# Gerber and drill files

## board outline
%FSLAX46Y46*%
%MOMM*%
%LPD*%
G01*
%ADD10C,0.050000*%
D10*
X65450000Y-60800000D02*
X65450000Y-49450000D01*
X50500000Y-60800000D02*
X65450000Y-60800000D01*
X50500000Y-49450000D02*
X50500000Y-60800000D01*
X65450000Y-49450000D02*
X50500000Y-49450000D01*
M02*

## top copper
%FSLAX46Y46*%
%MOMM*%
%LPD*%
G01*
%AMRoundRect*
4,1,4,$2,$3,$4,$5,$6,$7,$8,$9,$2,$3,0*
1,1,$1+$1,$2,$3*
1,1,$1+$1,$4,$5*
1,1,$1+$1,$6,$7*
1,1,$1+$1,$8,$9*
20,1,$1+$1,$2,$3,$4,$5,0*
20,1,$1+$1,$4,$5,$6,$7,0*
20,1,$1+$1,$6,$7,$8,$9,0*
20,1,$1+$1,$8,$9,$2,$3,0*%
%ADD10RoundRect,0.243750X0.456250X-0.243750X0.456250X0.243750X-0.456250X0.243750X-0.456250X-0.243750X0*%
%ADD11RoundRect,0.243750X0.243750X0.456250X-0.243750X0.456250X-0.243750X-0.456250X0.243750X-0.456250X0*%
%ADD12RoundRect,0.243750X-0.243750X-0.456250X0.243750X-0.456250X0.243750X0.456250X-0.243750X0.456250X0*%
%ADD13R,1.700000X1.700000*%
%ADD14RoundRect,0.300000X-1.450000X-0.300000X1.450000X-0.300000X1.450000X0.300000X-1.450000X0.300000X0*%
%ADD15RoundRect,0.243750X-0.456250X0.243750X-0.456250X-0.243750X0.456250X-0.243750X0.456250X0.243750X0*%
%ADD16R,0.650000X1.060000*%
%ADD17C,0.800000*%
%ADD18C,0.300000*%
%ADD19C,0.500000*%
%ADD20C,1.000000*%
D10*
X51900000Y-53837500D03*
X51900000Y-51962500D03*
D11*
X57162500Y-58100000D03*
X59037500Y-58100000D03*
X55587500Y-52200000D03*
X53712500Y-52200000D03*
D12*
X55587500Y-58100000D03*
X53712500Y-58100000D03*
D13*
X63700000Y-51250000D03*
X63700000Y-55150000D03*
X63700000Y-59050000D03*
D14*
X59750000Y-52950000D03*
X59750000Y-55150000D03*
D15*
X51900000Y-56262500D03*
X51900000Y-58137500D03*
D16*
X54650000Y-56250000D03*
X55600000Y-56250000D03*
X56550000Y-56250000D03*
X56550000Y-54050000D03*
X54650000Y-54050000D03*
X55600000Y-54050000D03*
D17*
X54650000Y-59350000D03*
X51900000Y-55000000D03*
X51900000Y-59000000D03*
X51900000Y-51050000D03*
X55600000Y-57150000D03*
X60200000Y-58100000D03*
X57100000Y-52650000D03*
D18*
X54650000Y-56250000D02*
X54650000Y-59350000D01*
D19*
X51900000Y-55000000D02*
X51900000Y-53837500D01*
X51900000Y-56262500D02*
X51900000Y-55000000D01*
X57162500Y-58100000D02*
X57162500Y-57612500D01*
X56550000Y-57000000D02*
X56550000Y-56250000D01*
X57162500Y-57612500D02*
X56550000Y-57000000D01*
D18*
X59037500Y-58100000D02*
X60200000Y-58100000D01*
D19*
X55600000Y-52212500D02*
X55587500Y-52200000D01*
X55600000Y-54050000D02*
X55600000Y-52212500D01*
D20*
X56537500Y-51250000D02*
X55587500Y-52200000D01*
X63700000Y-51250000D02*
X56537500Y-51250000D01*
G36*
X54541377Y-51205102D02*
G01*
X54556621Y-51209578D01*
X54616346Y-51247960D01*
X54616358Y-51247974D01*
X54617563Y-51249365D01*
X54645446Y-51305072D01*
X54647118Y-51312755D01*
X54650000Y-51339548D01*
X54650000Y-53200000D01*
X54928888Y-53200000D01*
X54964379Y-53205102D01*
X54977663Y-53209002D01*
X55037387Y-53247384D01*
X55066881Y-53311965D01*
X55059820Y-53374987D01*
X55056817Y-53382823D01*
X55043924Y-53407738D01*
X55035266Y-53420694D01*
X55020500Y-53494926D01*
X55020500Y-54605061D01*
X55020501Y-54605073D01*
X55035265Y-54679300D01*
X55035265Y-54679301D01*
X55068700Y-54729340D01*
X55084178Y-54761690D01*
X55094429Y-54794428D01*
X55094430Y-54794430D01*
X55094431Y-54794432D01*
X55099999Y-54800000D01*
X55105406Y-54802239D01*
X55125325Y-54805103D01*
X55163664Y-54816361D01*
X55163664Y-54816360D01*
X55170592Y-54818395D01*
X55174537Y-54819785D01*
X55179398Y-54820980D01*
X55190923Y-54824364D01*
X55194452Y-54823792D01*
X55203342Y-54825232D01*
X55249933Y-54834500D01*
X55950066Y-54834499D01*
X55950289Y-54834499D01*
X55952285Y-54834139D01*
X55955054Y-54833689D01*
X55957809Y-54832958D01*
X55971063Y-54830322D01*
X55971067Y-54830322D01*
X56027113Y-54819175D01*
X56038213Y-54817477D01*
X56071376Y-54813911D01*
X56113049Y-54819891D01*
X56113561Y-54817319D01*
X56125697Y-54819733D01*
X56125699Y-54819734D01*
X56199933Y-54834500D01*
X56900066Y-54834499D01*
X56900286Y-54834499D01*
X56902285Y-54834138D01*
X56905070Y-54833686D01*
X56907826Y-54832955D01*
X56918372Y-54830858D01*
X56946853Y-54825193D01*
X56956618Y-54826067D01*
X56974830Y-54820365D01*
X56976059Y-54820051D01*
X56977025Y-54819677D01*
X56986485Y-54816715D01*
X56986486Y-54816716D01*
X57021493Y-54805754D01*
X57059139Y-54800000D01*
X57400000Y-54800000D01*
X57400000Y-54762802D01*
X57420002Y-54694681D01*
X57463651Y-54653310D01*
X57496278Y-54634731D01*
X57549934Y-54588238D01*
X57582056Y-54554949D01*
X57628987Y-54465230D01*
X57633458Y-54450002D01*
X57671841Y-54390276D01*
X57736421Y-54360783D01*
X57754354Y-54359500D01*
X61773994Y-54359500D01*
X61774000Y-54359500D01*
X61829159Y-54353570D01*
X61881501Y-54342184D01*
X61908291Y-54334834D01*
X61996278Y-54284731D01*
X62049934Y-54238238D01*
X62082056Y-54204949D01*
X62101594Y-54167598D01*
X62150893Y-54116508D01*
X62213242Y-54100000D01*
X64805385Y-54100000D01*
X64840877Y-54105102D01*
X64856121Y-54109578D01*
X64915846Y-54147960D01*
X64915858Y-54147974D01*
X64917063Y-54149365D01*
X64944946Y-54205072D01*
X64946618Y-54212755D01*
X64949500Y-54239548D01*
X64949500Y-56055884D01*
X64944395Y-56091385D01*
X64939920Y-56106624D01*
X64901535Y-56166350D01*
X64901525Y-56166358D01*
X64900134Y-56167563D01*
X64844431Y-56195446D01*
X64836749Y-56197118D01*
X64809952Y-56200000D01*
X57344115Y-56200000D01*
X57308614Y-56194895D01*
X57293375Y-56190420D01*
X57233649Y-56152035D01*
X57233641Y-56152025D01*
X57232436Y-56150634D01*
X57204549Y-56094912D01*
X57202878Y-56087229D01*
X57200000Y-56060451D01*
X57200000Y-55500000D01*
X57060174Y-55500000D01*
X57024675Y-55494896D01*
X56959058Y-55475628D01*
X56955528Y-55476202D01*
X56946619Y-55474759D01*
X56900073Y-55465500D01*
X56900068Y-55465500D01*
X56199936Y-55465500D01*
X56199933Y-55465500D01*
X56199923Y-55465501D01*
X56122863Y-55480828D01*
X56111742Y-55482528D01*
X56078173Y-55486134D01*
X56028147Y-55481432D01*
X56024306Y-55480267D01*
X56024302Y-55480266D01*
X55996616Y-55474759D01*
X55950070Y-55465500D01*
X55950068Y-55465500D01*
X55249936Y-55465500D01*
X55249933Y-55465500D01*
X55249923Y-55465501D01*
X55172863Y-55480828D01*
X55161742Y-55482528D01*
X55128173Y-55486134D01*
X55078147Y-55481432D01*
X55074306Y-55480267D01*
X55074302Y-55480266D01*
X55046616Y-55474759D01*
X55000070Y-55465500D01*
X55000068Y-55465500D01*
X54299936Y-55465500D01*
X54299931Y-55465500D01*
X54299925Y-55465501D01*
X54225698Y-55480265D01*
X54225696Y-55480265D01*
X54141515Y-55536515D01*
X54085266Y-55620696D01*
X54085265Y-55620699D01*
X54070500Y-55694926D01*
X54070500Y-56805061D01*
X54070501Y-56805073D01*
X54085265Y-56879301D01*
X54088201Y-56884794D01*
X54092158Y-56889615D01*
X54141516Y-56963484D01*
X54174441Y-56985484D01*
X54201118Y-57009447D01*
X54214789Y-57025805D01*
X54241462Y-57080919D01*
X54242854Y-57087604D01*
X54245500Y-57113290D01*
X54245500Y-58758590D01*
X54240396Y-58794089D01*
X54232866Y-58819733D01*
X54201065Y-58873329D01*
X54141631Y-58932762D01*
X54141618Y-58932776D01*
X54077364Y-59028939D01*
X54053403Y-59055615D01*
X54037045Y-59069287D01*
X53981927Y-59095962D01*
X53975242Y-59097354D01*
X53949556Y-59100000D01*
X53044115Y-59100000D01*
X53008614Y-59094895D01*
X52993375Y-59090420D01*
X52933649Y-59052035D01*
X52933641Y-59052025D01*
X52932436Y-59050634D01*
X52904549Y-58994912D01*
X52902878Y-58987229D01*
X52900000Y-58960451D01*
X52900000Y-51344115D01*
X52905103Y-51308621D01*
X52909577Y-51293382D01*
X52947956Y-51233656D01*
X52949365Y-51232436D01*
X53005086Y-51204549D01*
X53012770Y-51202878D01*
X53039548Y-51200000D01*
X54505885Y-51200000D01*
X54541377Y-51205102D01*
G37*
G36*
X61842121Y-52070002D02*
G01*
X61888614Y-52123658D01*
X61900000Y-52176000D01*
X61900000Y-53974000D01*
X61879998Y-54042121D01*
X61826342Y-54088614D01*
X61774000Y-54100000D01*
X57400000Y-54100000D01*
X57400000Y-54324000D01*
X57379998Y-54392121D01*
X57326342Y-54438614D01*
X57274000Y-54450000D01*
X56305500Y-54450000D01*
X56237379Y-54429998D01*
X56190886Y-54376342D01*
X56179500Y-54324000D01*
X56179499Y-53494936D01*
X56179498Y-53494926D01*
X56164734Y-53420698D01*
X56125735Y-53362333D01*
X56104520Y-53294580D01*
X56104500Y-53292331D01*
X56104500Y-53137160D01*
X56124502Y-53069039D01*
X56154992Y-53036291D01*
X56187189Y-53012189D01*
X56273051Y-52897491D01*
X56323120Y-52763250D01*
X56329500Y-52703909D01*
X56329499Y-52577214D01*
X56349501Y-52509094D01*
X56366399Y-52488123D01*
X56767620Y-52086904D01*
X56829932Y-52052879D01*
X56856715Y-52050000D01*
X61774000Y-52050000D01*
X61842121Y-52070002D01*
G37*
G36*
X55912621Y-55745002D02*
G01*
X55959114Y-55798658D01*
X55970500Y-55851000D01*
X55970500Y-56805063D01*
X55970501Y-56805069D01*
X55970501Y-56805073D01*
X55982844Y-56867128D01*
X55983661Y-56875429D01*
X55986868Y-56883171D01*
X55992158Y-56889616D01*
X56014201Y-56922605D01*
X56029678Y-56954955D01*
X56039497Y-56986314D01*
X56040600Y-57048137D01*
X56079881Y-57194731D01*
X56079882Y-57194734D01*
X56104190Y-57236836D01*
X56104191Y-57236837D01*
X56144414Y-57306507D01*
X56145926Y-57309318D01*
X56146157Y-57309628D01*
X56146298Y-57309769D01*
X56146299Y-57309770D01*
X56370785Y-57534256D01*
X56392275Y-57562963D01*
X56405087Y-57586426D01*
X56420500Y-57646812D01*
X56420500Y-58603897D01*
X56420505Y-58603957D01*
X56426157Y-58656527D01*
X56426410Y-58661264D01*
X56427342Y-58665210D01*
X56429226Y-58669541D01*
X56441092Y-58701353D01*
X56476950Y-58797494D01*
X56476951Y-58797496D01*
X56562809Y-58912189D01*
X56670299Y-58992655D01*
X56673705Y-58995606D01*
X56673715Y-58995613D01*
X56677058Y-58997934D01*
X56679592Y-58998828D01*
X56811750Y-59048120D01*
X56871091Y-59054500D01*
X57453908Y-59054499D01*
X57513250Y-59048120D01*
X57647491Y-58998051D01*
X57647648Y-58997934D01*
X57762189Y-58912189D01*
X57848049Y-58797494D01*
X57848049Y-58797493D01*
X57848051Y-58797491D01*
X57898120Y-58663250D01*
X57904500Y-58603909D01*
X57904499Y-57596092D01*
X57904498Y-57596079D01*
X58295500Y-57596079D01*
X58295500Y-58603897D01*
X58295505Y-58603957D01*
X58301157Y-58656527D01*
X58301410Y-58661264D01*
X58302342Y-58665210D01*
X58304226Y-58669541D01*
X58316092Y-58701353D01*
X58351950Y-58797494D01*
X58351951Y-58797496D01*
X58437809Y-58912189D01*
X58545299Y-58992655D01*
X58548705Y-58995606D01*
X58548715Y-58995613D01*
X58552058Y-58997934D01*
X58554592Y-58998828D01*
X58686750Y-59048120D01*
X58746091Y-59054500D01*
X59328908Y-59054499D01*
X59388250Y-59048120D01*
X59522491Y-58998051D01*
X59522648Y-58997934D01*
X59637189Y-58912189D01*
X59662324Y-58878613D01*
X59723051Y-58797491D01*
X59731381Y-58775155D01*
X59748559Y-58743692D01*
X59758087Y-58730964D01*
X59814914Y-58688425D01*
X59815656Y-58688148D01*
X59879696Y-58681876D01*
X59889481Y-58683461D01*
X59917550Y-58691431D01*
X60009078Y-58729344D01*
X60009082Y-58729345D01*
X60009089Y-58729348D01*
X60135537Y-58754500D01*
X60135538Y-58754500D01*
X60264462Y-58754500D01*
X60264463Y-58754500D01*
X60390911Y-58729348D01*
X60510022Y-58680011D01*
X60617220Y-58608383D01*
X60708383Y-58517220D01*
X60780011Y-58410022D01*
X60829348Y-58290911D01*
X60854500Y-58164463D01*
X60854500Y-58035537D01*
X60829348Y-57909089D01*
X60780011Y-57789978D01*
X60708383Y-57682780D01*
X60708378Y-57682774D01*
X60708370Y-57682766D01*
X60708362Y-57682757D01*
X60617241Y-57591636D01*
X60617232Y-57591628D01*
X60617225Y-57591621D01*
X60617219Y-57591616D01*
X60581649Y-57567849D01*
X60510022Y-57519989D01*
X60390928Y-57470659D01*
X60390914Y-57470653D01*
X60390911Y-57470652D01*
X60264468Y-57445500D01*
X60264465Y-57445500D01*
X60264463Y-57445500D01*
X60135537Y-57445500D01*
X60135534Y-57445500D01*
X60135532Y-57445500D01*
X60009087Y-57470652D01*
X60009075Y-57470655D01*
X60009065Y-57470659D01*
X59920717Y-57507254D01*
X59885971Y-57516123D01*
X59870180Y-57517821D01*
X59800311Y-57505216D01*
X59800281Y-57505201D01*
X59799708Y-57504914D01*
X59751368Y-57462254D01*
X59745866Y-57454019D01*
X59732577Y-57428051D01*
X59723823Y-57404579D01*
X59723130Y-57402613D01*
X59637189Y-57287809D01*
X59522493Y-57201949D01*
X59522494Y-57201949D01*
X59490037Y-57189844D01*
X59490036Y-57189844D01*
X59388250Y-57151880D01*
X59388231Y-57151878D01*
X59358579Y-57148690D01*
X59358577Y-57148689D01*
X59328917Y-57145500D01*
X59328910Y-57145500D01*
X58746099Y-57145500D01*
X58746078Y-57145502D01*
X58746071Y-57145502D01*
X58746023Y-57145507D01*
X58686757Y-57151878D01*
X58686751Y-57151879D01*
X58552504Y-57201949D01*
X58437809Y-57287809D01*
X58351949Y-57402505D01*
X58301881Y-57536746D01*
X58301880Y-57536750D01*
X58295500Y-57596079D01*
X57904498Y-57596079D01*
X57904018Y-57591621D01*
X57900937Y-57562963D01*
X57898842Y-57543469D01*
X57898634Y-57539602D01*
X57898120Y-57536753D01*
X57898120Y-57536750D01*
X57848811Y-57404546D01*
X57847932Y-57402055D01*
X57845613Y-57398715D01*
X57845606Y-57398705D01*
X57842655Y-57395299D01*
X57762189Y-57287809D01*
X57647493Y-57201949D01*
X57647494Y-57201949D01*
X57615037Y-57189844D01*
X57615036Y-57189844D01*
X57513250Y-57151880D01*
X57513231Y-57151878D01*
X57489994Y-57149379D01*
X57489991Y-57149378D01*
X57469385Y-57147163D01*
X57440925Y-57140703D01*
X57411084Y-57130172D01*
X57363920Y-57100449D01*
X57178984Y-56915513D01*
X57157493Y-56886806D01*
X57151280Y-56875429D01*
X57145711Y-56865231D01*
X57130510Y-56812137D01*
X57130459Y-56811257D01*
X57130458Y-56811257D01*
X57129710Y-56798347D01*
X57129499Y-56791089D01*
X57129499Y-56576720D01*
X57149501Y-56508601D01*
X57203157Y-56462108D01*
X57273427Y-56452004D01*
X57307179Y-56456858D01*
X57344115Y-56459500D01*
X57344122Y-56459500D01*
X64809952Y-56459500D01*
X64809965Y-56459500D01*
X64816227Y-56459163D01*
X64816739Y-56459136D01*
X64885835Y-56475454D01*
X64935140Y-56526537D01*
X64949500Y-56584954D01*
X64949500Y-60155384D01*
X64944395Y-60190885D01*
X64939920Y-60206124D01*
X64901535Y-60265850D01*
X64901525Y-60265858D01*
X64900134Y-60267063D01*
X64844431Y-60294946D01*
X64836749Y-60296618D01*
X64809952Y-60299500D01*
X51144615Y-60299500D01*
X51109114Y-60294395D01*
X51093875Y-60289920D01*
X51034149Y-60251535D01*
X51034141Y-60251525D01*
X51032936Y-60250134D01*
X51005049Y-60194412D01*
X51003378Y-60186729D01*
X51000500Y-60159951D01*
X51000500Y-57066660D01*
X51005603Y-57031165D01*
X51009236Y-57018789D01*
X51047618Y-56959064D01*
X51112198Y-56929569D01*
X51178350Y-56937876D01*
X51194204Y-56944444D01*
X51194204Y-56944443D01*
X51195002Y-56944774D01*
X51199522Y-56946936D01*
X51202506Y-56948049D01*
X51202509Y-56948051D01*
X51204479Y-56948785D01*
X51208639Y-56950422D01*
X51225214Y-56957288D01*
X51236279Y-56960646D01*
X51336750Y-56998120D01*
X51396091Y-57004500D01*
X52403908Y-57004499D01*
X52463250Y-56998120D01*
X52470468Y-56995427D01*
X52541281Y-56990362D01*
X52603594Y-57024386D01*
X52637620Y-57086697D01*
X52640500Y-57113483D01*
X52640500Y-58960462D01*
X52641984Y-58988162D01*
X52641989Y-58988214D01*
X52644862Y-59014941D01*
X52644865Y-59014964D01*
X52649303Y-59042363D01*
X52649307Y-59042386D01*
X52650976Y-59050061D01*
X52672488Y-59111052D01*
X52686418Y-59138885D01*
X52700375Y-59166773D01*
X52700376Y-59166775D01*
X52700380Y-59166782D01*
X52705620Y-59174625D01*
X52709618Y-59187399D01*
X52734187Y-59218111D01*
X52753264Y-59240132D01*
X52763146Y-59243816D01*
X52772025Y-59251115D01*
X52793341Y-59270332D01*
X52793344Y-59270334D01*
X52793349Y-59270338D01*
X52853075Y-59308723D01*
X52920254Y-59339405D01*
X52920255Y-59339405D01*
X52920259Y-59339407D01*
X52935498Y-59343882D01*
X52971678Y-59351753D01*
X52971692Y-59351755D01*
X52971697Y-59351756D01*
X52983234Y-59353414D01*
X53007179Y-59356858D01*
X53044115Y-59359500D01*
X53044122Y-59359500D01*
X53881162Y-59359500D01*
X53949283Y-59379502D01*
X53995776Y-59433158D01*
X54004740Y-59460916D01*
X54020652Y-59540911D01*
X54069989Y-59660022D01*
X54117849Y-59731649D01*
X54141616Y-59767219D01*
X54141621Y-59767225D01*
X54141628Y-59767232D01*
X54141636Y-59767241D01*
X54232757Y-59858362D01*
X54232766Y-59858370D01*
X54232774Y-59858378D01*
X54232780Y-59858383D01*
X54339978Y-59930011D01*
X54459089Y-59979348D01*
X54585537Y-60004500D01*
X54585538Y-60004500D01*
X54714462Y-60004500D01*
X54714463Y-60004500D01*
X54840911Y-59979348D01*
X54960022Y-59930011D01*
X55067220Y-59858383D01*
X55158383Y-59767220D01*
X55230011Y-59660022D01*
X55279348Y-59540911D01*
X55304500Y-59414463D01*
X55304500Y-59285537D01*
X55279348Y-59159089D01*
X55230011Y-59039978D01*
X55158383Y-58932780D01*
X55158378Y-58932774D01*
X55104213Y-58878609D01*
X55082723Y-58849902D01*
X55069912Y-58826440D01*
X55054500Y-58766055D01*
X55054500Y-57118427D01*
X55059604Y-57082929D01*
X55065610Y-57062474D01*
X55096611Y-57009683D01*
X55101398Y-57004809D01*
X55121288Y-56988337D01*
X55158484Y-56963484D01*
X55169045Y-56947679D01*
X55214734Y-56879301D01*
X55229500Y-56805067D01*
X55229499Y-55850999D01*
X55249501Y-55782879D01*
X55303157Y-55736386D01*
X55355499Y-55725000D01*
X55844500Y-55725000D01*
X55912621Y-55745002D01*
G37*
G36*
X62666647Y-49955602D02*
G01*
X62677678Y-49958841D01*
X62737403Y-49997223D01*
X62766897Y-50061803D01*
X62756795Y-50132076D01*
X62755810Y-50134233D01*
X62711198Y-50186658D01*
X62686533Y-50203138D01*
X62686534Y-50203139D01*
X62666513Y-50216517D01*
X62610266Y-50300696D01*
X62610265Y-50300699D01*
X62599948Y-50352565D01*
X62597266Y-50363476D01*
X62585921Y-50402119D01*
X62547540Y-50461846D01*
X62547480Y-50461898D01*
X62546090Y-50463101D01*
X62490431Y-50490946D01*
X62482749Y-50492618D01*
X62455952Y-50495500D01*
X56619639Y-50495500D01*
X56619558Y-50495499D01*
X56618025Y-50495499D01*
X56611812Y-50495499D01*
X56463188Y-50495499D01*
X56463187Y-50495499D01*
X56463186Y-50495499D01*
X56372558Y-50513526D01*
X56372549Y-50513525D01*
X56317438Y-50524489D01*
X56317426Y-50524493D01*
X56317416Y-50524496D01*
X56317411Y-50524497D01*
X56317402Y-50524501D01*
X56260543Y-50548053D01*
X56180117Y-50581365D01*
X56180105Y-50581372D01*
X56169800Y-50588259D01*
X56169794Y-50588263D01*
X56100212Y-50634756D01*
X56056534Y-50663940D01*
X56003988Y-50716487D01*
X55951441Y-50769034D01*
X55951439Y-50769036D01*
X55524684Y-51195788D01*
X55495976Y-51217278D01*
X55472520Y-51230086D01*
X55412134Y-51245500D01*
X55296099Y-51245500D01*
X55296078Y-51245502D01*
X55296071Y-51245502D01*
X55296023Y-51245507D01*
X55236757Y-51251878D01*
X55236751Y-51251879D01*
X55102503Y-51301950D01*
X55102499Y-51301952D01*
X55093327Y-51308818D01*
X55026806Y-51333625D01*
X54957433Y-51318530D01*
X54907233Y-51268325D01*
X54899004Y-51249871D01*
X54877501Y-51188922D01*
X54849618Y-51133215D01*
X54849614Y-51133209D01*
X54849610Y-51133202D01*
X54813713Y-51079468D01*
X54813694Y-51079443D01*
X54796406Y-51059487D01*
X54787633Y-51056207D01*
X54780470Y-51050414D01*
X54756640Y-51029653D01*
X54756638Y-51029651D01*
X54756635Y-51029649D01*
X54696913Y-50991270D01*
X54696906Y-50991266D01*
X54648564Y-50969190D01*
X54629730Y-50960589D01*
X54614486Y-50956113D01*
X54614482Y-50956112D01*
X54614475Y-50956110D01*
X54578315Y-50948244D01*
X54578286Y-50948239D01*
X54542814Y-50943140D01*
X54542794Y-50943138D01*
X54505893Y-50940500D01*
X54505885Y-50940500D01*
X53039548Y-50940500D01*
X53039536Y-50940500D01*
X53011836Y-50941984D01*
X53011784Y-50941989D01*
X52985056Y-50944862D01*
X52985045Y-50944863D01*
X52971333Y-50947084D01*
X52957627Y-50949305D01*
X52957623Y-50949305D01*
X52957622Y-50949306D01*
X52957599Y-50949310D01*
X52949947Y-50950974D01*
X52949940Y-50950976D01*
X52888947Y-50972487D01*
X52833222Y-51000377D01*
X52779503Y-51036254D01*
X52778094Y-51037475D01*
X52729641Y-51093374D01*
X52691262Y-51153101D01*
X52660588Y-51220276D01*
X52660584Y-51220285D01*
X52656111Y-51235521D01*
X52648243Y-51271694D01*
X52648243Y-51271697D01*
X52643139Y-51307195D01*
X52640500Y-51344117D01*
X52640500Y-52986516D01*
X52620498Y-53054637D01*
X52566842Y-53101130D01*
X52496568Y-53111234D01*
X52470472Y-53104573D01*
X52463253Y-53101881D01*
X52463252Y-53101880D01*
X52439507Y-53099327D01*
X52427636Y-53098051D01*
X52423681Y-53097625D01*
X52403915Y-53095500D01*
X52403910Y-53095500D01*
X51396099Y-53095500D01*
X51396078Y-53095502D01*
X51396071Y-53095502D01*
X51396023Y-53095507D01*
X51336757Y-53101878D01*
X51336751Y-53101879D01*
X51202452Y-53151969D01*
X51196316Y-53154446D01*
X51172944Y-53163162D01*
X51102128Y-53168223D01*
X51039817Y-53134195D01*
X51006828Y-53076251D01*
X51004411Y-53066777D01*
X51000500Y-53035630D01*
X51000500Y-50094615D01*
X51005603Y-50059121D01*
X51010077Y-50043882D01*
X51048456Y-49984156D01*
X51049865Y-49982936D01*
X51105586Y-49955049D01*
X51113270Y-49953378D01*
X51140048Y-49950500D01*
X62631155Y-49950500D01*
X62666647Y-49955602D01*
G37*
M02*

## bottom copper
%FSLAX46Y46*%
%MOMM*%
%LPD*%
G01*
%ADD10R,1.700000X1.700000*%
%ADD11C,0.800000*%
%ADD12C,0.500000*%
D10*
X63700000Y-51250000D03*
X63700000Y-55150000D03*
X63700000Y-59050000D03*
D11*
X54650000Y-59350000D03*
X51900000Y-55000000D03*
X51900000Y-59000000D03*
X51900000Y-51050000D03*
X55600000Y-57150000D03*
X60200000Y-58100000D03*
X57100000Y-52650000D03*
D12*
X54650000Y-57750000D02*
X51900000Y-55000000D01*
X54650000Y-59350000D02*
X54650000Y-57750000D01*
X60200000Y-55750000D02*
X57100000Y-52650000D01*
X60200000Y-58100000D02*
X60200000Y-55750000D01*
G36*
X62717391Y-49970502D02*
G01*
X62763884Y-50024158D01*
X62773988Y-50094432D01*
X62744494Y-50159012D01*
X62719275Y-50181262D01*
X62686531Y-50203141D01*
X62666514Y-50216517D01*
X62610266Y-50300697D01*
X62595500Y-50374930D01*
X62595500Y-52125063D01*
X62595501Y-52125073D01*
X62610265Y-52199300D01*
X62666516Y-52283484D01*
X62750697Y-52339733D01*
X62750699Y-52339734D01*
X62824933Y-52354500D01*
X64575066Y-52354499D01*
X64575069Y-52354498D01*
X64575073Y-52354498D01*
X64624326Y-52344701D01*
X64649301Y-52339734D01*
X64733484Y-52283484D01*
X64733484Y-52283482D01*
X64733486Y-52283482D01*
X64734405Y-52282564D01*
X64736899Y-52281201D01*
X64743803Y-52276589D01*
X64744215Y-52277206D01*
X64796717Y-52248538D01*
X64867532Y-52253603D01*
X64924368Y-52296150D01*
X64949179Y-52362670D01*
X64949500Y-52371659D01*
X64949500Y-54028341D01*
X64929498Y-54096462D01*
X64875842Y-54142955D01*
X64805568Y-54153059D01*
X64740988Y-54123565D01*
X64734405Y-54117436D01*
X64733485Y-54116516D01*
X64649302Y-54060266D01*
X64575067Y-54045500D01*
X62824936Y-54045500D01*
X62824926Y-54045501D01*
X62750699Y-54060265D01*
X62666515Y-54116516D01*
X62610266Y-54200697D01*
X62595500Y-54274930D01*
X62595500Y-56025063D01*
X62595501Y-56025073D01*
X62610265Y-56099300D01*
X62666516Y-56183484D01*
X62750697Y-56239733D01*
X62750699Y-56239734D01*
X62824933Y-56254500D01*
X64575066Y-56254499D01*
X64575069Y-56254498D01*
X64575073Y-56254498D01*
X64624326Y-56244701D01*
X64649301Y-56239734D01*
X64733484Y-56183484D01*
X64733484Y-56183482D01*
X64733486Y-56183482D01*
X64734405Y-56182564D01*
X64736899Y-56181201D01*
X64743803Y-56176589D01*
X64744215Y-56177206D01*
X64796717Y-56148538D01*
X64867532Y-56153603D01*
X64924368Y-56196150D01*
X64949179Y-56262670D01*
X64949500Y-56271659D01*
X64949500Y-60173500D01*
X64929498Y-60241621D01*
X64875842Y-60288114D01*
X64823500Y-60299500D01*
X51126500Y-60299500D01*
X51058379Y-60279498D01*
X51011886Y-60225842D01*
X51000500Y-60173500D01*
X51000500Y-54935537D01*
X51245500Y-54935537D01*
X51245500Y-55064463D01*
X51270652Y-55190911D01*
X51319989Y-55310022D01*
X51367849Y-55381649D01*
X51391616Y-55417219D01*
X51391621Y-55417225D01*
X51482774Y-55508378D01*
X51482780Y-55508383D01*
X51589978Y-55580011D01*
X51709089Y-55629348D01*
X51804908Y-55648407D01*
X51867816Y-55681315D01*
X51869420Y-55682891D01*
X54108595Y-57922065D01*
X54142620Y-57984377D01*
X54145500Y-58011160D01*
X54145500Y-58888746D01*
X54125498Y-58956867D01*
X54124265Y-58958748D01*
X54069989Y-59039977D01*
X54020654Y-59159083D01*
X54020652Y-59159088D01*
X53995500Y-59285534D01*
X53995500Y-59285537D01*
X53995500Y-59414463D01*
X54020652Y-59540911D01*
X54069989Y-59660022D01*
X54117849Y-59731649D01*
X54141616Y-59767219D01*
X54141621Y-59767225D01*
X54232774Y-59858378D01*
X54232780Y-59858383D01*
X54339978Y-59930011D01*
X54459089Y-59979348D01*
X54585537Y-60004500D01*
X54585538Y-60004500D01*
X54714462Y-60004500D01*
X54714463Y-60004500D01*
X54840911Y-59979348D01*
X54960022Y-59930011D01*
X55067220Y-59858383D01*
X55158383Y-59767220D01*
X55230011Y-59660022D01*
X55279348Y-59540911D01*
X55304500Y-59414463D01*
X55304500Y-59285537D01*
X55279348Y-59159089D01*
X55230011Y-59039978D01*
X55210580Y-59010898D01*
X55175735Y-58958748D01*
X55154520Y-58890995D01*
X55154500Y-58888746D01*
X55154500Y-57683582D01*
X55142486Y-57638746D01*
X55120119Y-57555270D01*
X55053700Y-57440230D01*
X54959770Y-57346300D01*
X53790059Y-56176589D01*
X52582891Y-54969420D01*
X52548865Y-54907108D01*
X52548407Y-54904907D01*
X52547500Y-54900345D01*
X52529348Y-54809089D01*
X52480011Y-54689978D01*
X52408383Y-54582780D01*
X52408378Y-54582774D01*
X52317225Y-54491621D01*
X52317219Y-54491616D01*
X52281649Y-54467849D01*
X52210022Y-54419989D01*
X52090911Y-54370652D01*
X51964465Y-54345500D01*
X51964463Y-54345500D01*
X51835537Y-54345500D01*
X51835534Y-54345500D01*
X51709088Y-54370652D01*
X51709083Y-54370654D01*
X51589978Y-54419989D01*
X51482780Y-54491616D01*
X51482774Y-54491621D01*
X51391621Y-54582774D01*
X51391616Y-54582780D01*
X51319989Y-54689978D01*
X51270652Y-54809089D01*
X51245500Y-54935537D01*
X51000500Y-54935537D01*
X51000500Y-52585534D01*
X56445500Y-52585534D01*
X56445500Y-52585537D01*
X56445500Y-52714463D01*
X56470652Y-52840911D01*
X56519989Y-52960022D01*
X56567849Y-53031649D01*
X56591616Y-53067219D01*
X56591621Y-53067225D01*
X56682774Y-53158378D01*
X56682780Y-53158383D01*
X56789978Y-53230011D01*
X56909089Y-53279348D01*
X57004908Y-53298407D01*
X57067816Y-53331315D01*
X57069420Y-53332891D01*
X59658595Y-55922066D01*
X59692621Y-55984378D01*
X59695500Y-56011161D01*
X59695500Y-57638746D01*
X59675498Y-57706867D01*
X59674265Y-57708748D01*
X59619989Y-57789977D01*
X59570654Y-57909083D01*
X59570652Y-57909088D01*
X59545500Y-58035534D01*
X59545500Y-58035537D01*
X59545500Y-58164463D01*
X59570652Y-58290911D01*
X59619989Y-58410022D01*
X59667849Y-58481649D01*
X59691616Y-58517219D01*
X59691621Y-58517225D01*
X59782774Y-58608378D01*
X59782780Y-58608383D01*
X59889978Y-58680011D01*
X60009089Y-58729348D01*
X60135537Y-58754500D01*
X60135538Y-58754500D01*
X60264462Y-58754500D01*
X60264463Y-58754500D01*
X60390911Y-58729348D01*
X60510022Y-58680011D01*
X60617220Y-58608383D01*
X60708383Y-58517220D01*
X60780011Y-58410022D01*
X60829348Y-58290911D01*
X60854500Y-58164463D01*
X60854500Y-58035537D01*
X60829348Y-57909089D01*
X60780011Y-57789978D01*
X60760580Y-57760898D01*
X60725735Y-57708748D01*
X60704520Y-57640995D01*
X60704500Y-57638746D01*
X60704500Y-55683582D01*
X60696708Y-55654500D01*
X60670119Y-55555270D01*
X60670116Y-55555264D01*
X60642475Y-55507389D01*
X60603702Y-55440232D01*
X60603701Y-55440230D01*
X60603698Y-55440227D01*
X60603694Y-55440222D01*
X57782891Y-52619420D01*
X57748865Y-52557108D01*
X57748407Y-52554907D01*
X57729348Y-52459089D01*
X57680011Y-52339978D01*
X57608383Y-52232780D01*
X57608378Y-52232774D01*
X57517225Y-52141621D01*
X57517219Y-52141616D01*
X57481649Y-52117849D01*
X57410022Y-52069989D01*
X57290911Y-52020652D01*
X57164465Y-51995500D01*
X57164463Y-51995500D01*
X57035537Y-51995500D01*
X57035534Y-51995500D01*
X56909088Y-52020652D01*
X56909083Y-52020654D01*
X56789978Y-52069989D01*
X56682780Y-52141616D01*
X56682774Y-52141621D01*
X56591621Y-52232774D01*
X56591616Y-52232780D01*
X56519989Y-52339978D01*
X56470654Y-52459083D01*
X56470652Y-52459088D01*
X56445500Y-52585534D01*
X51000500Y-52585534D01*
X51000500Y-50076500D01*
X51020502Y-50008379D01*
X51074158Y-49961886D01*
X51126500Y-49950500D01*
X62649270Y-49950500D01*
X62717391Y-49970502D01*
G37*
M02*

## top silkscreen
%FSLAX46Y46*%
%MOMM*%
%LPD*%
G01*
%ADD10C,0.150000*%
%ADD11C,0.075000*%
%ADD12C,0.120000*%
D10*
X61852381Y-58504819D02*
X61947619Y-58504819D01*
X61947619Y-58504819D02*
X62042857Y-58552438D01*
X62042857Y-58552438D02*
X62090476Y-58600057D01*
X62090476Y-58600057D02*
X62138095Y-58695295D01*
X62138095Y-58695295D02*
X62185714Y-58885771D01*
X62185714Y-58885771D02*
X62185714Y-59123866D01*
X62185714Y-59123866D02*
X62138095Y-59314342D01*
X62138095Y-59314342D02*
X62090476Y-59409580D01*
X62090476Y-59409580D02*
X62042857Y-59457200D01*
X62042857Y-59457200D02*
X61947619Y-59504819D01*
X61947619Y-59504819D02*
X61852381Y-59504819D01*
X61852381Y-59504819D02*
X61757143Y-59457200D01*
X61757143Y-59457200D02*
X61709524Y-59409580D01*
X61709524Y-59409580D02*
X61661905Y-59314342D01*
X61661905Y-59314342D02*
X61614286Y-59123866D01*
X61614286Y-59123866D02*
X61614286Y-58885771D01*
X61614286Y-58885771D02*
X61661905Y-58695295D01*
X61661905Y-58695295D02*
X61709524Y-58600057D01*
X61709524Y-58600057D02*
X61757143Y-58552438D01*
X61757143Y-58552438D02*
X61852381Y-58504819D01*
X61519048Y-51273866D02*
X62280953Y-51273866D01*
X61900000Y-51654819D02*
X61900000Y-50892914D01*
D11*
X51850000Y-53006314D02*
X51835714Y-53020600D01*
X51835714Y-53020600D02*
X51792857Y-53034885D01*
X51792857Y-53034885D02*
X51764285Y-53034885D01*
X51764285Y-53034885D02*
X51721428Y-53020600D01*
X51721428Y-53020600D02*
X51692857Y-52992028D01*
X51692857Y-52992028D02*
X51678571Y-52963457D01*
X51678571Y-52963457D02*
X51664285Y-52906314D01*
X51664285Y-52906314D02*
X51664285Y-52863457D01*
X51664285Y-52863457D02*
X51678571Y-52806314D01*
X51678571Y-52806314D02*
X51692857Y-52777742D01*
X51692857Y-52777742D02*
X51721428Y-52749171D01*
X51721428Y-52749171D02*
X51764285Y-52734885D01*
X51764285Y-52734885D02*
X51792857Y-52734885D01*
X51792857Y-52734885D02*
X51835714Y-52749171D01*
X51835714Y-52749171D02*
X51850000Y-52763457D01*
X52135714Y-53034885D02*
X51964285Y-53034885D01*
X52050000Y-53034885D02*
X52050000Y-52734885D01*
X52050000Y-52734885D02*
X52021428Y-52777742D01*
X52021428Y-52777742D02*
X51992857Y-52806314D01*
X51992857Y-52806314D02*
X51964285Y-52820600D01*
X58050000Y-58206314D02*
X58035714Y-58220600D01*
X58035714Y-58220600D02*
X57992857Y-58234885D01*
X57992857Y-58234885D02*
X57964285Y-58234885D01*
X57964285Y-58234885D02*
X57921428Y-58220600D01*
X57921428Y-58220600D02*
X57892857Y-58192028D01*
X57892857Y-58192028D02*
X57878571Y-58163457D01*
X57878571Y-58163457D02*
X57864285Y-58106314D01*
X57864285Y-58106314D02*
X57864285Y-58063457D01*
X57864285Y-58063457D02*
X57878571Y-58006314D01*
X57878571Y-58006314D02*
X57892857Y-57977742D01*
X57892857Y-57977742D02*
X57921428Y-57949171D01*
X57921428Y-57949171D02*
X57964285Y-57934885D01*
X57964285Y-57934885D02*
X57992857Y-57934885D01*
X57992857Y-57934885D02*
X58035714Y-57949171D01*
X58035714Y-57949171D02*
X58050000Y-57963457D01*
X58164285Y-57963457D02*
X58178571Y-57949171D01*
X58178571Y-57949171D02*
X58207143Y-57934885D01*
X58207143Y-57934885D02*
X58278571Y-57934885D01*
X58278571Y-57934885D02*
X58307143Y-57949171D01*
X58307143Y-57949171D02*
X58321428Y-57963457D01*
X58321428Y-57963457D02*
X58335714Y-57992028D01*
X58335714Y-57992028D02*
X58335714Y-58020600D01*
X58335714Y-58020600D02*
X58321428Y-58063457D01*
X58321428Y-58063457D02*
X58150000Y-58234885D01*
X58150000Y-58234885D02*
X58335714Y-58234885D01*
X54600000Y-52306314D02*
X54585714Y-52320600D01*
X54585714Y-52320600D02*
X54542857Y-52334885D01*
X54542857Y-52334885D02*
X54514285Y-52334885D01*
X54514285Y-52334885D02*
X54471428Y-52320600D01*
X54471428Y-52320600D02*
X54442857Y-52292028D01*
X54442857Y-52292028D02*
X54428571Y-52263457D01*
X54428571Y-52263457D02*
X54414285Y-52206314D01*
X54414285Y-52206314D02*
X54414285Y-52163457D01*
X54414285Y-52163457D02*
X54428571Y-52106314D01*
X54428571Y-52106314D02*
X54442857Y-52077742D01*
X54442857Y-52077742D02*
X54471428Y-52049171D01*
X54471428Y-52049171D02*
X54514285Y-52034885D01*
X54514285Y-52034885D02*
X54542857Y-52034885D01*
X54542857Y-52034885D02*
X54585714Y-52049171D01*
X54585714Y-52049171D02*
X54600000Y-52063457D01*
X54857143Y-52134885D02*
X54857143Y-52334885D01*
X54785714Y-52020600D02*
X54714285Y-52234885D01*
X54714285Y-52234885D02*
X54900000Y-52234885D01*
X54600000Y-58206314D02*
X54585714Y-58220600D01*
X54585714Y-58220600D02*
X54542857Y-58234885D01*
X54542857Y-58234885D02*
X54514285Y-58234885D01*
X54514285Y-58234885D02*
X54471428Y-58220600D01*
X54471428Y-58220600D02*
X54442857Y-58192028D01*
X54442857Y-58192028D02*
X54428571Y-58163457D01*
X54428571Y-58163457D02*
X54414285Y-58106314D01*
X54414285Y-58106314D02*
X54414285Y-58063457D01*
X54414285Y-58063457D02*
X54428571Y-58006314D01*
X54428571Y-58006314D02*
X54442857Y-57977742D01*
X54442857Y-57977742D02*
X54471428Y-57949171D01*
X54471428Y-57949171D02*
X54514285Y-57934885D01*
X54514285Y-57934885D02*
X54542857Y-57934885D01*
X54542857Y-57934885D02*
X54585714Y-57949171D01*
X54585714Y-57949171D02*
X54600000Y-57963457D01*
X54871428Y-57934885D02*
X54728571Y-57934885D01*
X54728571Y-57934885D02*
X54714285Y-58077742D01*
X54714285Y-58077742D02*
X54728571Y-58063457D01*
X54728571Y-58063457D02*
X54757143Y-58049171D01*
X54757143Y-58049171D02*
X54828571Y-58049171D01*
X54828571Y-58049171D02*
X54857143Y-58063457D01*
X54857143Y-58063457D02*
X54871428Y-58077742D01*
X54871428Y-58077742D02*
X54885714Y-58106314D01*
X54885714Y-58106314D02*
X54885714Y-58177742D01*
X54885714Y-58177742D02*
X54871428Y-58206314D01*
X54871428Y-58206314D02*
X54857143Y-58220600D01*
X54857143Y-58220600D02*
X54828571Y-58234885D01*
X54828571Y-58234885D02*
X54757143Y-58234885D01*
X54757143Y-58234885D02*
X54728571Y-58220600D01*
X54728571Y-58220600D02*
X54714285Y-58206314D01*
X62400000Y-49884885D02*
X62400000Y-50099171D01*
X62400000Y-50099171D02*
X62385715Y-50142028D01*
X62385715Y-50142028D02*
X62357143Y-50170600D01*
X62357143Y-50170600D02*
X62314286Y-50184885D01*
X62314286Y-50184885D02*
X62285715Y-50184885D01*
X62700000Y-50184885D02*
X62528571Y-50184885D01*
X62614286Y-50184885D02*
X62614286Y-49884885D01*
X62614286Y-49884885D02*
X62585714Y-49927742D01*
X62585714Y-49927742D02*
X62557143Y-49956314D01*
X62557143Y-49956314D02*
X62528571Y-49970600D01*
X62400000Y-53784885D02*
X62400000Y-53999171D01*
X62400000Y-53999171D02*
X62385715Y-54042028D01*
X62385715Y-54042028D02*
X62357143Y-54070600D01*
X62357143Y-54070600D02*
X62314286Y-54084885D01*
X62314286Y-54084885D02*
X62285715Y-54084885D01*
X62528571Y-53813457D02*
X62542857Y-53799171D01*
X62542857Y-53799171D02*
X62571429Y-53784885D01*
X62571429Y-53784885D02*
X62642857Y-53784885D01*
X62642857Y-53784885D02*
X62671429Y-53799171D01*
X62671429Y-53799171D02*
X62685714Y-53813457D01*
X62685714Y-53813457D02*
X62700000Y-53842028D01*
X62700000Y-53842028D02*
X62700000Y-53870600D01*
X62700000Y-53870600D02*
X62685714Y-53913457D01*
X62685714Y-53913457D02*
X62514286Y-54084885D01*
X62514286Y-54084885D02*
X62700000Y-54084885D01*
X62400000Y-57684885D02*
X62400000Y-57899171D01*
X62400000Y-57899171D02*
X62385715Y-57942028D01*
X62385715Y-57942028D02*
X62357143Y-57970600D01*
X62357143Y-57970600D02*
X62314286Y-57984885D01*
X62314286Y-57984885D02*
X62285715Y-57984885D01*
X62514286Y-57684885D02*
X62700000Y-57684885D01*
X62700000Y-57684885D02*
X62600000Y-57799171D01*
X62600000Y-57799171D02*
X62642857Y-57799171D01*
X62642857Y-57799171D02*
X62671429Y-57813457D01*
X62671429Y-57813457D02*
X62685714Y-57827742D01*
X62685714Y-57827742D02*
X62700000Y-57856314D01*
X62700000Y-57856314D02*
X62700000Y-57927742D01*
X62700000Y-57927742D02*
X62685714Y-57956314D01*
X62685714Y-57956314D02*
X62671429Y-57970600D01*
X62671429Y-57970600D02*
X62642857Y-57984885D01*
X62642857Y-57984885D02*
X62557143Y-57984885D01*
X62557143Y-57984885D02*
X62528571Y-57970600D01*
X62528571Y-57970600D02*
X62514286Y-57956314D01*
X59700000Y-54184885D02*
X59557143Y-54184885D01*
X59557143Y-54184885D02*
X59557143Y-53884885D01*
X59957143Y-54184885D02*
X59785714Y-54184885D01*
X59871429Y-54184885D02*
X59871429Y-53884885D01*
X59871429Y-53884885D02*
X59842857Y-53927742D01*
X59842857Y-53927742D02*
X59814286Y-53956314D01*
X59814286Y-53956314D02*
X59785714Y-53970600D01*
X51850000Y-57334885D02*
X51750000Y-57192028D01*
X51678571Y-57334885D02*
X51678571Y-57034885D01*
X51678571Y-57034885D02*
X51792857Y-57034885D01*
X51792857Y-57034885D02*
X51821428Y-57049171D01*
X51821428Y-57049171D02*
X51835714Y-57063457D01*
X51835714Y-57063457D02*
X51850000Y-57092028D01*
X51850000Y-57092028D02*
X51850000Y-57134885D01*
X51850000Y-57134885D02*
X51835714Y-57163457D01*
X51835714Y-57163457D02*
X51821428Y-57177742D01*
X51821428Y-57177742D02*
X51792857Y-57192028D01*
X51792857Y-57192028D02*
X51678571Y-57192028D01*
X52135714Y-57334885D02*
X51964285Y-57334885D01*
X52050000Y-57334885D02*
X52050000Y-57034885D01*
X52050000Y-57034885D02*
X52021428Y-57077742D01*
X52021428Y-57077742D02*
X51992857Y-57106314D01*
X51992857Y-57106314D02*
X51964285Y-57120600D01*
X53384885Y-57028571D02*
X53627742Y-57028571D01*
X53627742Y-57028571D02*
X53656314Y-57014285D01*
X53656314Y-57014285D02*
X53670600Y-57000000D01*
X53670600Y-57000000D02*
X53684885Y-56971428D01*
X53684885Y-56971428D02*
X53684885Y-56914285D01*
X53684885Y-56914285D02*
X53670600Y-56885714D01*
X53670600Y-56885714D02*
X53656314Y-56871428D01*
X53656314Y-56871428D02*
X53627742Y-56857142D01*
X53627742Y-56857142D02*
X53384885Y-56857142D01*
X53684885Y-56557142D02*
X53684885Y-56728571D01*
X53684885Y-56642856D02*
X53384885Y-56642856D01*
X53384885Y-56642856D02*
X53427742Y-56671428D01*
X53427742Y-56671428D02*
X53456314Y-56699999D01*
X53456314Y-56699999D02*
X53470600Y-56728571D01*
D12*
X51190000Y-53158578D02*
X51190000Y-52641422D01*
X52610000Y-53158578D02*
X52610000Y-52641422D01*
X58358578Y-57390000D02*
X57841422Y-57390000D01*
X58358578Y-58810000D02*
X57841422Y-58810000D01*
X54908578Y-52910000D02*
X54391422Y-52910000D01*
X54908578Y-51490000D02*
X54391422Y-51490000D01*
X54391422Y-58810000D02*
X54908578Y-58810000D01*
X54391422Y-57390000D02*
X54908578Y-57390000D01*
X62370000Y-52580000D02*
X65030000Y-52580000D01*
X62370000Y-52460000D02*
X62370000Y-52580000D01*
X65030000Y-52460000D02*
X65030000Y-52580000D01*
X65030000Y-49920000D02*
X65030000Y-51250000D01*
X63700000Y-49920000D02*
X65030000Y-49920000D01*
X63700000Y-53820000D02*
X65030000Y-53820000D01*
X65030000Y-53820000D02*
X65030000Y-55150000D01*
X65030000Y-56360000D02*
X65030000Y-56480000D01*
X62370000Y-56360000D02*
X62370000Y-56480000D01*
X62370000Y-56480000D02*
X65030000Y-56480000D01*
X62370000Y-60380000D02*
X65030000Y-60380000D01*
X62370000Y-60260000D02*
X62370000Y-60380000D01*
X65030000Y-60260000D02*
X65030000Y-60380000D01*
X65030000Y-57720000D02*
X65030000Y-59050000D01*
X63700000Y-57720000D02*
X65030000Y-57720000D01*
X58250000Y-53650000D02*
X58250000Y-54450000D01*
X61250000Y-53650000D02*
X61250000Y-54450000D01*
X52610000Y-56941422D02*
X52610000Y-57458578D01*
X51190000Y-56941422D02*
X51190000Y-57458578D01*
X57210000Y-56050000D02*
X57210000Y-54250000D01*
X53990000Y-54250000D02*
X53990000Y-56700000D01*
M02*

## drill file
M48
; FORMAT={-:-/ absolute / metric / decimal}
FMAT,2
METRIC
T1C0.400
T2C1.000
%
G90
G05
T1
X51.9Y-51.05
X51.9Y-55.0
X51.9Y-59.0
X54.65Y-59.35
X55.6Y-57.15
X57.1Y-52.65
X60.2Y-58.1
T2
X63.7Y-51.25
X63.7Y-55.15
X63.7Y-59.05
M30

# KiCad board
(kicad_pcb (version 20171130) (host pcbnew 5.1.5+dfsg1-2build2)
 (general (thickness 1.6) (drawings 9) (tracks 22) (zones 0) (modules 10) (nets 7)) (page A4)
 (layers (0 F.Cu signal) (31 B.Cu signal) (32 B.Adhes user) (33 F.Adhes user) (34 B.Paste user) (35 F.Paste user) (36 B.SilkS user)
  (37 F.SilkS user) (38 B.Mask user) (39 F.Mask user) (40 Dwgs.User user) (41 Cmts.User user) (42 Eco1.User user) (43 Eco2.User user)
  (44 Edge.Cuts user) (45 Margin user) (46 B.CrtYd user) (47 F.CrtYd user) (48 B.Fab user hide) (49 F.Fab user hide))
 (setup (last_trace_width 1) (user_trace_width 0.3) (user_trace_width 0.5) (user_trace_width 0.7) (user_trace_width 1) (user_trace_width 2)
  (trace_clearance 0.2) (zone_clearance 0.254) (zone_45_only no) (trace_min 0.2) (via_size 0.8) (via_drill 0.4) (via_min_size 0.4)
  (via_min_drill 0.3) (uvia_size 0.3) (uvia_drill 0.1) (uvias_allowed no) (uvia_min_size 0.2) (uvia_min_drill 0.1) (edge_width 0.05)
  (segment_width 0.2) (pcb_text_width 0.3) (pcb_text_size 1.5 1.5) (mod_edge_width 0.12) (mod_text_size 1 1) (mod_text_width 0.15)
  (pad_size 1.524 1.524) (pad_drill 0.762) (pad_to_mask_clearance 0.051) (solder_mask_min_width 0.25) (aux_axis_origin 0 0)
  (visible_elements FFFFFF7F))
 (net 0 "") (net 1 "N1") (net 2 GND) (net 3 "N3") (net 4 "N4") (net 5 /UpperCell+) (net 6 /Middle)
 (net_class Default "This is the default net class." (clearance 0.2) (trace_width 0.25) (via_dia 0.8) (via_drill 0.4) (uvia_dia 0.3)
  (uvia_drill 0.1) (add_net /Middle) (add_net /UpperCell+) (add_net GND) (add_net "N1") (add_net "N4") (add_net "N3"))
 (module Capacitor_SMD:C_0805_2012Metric (layer F.Cu) (at 51.9 52.9 90)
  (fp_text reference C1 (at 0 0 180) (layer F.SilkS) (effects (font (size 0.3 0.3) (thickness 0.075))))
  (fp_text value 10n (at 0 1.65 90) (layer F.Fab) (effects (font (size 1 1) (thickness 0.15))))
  (fp_line (start -0.258578 -0.71) (end 0.258578 -0.71) (layer F.SilkS) (width 0.12))
  (fp_line (start -0.258578 0.71) (end 0.258578 0.71) (layer F.SilkS) (width 0.12))
  (pad 1 smd roundrect (at -0.9375 0 90) (size 0.975 1.4) (layers F.Cu F.Paste F.Mask) (roundrect_rratio 0.25) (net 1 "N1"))
  (pad 2 smd roundrect (at 0.9375 0 90) (size 0.975 1.4) (layers F.Cu F.Paste F.Mask) (roundrect_rratio 0.25) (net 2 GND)))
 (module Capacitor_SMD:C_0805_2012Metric (layer F.Cu) (at 58.1 58.1 180)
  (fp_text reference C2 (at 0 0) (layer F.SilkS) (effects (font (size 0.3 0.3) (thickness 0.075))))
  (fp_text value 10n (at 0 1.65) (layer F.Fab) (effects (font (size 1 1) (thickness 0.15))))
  (fp_line (start -0.258578 0.71) (end 0.258578 0.71) (layer F.SilkS) (width 0.12))
  (fp_line (start -0.258578 -0.71) (end 0.258578 -0.71) (layer F.SilkS) (width 0.12))
  (pad 2 smd roundrect (at 0.9375 0 180) (size 0.975 1.4) (layers F.Cu F.Paste F.Mask) (roundrect_rratio 0.25) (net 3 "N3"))
  (pad 1 smd roundrect (at -0.9375 0 180) (size 0.975 1.4) (layers F.Cu F.Paste F.Mask) (roundrect_rratio 0.25) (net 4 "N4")))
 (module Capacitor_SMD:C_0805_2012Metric (layer F.Cu) (at 54.65 52.2 180)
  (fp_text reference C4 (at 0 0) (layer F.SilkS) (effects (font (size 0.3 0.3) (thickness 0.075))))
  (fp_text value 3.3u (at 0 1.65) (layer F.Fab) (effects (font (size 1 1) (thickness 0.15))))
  (fp_line (start -0.258578 -0.71) (end 0.258578 -0.71) (layer F.SilkS) (width 0.12))
  (fp_line (start -0.258578 0.71) (end 0.258578 0.71) (layer F.SilkS) (width 0.12))
  (pad 1 smd roundrect (at -0.9375 0 180) (size 0.975 1.4) (layers F.Cu F.Paste F.Mask) (roundrect_rratio 0.25) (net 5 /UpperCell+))
  (pad 2 smd roundrect (at 0.9375 0 180) (size 0.975 1.4) (layers F.Cu F.Paste F.Mask) (roundrect_rratio 0.25) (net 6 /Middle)))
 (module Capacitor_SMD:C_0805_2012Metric (layer F.Cu) (at 54.65 58.1)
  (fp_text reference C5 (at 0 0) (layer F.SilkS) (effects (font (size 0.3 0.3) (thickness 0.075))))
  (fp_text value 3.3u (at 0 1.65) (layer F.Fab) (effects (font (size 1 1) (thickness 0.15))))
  (fp_line (start -0.258578 0.71) (end 0.258578 0.71) (layer F.SilkS) (width 0.12))
  (fp_line (start -0.258578 -0.71) (end 0.258578 -0.71) (layer F.SilkS) (width 0.12))
  (pad 2 smd roundrect (at 0.9375 0) (size 0.975 1.4) (layers F.Cu F.Paste F.Mask) (roundrect_rratio 0.25) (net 2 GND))
  (pad 1 smd roundrect (at -0.9375 0) (size 0.975 1.4) (layers F.Cu F.Paste F.Mask) (roundrect_rratio 0.25) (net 6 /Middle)))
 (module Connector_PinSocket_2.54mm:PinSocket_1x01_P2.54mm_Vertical (layer F.Cu) (at 63.7 51.25)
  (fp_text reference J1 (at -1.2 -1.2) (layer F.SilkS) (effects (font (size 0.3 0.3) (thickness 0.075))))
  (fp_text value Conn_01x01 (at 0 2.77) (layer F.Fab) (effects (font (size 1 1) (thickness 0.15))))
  (fp_line (start -1.33 1.33) (end 1.33 1.33) (layer F.SilkS) (width 0.12))
  (fp_line (start -1.33 1.21) (end -1.33 1.33) (layer F.SilkS) (width 0.12))
  (fp_line (start 1.33 1.21) (end 1.33 1.33) (layer F.SilkS) (width 0.12))
  (fp_line (start 1.33 -1.33) (end 1.33 0) (layer F.SilkS) (width 0.12))
  (fp_line (start 0 -1.33) (end 1.33 -1.33) (layer F.SilkS) (width 0.12))
  (pad 1 thru_hole rect (at 0 0) (size 1.7 1.7) (drill 1) (layers *.Cu *.Mask) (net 5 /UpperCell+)))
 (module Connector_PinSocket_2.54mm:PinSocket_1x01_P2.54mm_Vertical (layer F.Cu) (at 63.7 55.15)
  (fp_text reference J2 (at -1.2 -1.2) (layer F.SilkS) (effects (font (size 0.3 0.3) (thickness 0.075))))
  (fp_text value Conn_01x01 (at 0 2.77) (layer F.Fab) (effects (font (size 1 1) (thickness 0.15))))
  (fp_line (start 0 -1.33) (end 1.33 -1.33) (layer F.SilkS) (width 0.12))
  (fp_line (start 1.33 -1.33) (end 1.33 0) (layer F.SilkS) (width 0.12))
  (fp_line (start 1.33 1.21) (end 1.33 1.33) (layer F.SilkS) (width 0.12))
  (fp_line (start -1.33 1.21) (end -1.33 1.33) (layer F.SilkS) (width 0.12))
  (fp_line (start -1.33 1.33) (end 1.33 1.33) (layer F.SilkS) (width 0.12))
  (pad 1 thru_hole rect (at 0 0) (size 1.7 1.7) (drill 1) (layers *.Cu *.Mask) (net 6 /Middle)))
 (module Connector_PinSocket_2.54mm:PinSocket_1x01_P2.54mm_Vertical (layer F.Cu) (at 63.7 59.05)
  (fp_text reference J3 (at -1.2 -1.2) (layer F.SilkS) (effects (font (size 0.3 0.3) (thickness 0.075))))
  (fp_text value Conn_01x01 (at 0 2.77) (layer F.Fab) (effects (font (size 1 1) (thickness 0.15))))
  (fp_line (start -1.33 1.33) (end 1.33 1.33) (layer F.SilkS) (width 0.12))
  (fp_line (start -1.33 1.21) (end -1.33 1.33) (layer F.SilkS) (width 0.12))
  (fp_line (start 1.33 1.21) (end 1.33 1.33) (layer F.SilkS) (width 0.12))
  (fp_line (start 1.33 -1.33) (end 1.33 0) (layer F.SilkS) (width 0.12))
  (fp_line (start 0 -1.33) (end 1.33 -1.33) (layer F.SilkS) (width 0.12))
  (pad 1 thru_hole rect (at 0 0) (size 1.7 1.7) (drill 1) (layers *.Cu *.Mask) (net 2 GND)))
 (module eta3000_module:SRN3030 (layer F.Cu) (at 59.75 54.05)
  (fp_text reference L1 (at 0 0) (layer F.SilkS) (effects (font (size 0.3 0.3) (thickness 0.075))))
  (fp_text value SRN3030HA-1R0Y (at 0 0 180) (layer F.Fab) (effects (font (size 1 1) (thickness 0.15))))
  (fp_line (start -1.5 -0.4) (end -1.5 0.4) (layer F.SilkS) (width 0.12))
  (fp_line (start 1.5 -0.4) (end 1.5 0.4) (layer F.SilkS) (width 0.12))
  (pad 1 smd roundrect (at 0 -1.1) (size 3.5 1.2) (layers F.Cu F.Paste F.Mask) (roundrect_rratio 0.25) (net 4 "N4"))
  (pad 2 smd roundrect (at 0 1.1) (size 3.5 1.2) (layers F.Cu F.Paste F.Mask) (roundrect_rratio 0.25) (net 6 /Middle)))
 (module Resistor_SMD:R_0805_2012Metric (layer F.Cu) (at 51.9 57.2 270)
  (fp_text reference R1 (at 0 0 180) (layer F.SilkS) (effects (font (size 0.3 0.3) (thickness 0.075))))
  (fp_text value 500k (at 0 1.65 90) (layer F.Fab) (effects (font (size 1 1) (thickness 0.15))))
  (fp_line (start -0.258578 -0.71) (end 0.258578 -0.71) (layer F.SilkS) (width 0.12))
  (fp_line (start -0.258578 0.71) (end 0.258578 0.71) (layer F.SilkS) (width 0.12))
  (pad 1 smd roundrect (at -0.9375 0 270) (size 0.975 1.4) (layers F.Cu F.Paste F.Mask) (roundrect_rratio 0.25) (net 1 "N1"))
  (pad 2 smd roundrect (at 0.9375 0 270) (size 0.975 1.4) (layers F.Cu F.Paste F.Mask) (roundrect_rratio 0.25) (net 2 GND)))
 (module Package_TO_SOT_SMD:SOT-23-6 (layer F.Cu) (at 55.6 55.15 90)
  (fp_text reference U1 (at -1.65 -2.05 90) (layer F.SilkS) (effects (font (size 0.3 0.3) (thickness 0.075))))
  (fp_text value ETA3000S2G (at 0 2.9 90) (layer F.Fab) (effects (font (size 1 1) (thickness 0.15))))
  (fp_line (start -0.9 1.61) (end 0.9 1.61) (layer F.SilkS) (width 0.12))
  (fp_line (start 0.9 -1.61) (end -1.55 -1.61) (layer F.SilkS) (width 0.12))
  (pad 1 smd rect (at -1.1 -0.95 90) (size 1.06 0.65) (layers F.Cu F.Paste F.Mask) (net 1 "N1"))
  (pad 2 smd rect (at -1.1 0 90) (size 1.06 0.65) (layers F.Cu F.Paste F.Mask) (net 2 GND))
  (pad 3 smd rect (at -1.1 0.95 90) (size 1.06 0.65) (layers F.Cu F.Paste F.Mask) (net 3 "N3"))
  (pad 4 smd rect (at 1.1 0.95 90) (size 1.06 0.65) (layers F.Cu F.Paste F.Mask) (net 4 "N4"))
  (pad 6 smd rect (at 1.1 -0.95 90) (size 1.06 0.65) (layers F.Cu F.Paste F.Mask) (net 6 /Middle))
  (pad 5 smd rect (at 1.1 0 90) (size 1.06 0.65) (layers F.Cu F.Paste F.Mask) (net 5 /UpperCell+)))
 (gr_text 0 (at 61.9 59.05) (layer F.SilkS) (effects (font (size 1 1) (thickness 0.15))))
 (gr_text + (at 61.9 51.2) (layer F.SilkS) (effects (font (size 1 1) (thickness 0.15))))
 (gr_line (start 65.45 60.8) (end 65.45 49.45) (layer Edge.Cuts) (width 0.05))
 (gr_line (start 50.5 60.8) (end 65.45 60.8) (layer Edge.Cuts) (width 0.05))
 (gr_line (start 50.5 49.45) (end 50.5 60.8) (layer Edge.Cuts) (width 0.05))
 (gr_line (start 65.45 49.45) (end 50.5 49.45) (layer Edge.Cuts) (width 0.05))
 (via (at 54.65 59.35) (size 0.8) (drill 0.4) (layers F.Cu B.Cu) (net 1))
 (segment (start 54.65 56.25) (end 54.65 59.35) (width 0.3) (layer F.Cu) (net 1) (status 10))
 (via (at 51.9 55) (size 0.8) (drill 0.4) (layers F.Cu B.Cu) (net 1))
 (segment (start 54.65 57.75) (end 51.9 55) (width 0.5) (layer B.Cu) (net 1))
 (segment (start 54.65 59.35) (end 54.65 57.75) (width 0.5) (layer B.Cu) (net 1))
 (segment (start 51.9 55) (end 51.9 53.8375) (width 0.5) (layer F.Cu) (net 1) (status 20))
 (segment (start 51.9 56.2625) (end 51.9 55) (width 0.5) (layer F.Cu) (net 1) (status 10))
 (via (at 51.9 59) (size 0.8) (drill 0.4) (layers F.Cu B.Cu) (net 2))
 (via (at 51.9 51.05) (size 0.8) (drill 0.4) (layers F.Cu B.Cu) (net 2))
 (via (at 55.6 57.15) (size 0.8) (drill 0.4) (layers F.Cu B.Cu) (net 2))
 (segment (start 57.1625 58.1) (end 57.1625 57.6125) (width 0.5) (layer F.Cu) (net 3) (status 30))
 (segment (start 56.55 57) (end 56.55 56.25) (width 0.5) (layer F.Cu) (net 3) (status 20))
 (segment (start 57.1625 57.6125) (end 56.55 57) (width 0.5) (layer F.Cu) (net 3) (status 10))
 (via (at 60.2 58.1) (size 0.8) (drill 0.4) (layers F.Cu B.Cu) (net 4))
 (segment (start 59.0375 58.1) (end 60.2 58.1) (width 0.3) (layer F.Cu) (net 4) (status 10))
 (via (at 57.1 52.65) (size 0.8) (drill 0.4) (layers F.Cu B.Cu) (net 4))
 (segment (start 60.2 55.75) (end 57.1 52.65) (width 0.5) (layer B.Cu) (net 4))
 (segment (start 60.2 58.1) (end 60.2 55.75) (width 0.5) (layer B.Cu) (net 4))
 (segment (start 55.6 52.2125) (end 55.5875 52.2) (width 0.5) (layer F.Cu) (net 5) (status 30))
 (segment (start 55.6 54.05) (end 55.6 52.2125) (width 0.5) (layer F.Cu) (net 5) (status 30))
 (segment (start 56.5375 51.25) (end 55.5875 52.2) (width 1) (layer F.Cu) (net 5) (status 20))
 (segment (start 63.7 51.25) (end 56.5375 51.25) (width 1) (layer F.Cu) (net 5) (status 10))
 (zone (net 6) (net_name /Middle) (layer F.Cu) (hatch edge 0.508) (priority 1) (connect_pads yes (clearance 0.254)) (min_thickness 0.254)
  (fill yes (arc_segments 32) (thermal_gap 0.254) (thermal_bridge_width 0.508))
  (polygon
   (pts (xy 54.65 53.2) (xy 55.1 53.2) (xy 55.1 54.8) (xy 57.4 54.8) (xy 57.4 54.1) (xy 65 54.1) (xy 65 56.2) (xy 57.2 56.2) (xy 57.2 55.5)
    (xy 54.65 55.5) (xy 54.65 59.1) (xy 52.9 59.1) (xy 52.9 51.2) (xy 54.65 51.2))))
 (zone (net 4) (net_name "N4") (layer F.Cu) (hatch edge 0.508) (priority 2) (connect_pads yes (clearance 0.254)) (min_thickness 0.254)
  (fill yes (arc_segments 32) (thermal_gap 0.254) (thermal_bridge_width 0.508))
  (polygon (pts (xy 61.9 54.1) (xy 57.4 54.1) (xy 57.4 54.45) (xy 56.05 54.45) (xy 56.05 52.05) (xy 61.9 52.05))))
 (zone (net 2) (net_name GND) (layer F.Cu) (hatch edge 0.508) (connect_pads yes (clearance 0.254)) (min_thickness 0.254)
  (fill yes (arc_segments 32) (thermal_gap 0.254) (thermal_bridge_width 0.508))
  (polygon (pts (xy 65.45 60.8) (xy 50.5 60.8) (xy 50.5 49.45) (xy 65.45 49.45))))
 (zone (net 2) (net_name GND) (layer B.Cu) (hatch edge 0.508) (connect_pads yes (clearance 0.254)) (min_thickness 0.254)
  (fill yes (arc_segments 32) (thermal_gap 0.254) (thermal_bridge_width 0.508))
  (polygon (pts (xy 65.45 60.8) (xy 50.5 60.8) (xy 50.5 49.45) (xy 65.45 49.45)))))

